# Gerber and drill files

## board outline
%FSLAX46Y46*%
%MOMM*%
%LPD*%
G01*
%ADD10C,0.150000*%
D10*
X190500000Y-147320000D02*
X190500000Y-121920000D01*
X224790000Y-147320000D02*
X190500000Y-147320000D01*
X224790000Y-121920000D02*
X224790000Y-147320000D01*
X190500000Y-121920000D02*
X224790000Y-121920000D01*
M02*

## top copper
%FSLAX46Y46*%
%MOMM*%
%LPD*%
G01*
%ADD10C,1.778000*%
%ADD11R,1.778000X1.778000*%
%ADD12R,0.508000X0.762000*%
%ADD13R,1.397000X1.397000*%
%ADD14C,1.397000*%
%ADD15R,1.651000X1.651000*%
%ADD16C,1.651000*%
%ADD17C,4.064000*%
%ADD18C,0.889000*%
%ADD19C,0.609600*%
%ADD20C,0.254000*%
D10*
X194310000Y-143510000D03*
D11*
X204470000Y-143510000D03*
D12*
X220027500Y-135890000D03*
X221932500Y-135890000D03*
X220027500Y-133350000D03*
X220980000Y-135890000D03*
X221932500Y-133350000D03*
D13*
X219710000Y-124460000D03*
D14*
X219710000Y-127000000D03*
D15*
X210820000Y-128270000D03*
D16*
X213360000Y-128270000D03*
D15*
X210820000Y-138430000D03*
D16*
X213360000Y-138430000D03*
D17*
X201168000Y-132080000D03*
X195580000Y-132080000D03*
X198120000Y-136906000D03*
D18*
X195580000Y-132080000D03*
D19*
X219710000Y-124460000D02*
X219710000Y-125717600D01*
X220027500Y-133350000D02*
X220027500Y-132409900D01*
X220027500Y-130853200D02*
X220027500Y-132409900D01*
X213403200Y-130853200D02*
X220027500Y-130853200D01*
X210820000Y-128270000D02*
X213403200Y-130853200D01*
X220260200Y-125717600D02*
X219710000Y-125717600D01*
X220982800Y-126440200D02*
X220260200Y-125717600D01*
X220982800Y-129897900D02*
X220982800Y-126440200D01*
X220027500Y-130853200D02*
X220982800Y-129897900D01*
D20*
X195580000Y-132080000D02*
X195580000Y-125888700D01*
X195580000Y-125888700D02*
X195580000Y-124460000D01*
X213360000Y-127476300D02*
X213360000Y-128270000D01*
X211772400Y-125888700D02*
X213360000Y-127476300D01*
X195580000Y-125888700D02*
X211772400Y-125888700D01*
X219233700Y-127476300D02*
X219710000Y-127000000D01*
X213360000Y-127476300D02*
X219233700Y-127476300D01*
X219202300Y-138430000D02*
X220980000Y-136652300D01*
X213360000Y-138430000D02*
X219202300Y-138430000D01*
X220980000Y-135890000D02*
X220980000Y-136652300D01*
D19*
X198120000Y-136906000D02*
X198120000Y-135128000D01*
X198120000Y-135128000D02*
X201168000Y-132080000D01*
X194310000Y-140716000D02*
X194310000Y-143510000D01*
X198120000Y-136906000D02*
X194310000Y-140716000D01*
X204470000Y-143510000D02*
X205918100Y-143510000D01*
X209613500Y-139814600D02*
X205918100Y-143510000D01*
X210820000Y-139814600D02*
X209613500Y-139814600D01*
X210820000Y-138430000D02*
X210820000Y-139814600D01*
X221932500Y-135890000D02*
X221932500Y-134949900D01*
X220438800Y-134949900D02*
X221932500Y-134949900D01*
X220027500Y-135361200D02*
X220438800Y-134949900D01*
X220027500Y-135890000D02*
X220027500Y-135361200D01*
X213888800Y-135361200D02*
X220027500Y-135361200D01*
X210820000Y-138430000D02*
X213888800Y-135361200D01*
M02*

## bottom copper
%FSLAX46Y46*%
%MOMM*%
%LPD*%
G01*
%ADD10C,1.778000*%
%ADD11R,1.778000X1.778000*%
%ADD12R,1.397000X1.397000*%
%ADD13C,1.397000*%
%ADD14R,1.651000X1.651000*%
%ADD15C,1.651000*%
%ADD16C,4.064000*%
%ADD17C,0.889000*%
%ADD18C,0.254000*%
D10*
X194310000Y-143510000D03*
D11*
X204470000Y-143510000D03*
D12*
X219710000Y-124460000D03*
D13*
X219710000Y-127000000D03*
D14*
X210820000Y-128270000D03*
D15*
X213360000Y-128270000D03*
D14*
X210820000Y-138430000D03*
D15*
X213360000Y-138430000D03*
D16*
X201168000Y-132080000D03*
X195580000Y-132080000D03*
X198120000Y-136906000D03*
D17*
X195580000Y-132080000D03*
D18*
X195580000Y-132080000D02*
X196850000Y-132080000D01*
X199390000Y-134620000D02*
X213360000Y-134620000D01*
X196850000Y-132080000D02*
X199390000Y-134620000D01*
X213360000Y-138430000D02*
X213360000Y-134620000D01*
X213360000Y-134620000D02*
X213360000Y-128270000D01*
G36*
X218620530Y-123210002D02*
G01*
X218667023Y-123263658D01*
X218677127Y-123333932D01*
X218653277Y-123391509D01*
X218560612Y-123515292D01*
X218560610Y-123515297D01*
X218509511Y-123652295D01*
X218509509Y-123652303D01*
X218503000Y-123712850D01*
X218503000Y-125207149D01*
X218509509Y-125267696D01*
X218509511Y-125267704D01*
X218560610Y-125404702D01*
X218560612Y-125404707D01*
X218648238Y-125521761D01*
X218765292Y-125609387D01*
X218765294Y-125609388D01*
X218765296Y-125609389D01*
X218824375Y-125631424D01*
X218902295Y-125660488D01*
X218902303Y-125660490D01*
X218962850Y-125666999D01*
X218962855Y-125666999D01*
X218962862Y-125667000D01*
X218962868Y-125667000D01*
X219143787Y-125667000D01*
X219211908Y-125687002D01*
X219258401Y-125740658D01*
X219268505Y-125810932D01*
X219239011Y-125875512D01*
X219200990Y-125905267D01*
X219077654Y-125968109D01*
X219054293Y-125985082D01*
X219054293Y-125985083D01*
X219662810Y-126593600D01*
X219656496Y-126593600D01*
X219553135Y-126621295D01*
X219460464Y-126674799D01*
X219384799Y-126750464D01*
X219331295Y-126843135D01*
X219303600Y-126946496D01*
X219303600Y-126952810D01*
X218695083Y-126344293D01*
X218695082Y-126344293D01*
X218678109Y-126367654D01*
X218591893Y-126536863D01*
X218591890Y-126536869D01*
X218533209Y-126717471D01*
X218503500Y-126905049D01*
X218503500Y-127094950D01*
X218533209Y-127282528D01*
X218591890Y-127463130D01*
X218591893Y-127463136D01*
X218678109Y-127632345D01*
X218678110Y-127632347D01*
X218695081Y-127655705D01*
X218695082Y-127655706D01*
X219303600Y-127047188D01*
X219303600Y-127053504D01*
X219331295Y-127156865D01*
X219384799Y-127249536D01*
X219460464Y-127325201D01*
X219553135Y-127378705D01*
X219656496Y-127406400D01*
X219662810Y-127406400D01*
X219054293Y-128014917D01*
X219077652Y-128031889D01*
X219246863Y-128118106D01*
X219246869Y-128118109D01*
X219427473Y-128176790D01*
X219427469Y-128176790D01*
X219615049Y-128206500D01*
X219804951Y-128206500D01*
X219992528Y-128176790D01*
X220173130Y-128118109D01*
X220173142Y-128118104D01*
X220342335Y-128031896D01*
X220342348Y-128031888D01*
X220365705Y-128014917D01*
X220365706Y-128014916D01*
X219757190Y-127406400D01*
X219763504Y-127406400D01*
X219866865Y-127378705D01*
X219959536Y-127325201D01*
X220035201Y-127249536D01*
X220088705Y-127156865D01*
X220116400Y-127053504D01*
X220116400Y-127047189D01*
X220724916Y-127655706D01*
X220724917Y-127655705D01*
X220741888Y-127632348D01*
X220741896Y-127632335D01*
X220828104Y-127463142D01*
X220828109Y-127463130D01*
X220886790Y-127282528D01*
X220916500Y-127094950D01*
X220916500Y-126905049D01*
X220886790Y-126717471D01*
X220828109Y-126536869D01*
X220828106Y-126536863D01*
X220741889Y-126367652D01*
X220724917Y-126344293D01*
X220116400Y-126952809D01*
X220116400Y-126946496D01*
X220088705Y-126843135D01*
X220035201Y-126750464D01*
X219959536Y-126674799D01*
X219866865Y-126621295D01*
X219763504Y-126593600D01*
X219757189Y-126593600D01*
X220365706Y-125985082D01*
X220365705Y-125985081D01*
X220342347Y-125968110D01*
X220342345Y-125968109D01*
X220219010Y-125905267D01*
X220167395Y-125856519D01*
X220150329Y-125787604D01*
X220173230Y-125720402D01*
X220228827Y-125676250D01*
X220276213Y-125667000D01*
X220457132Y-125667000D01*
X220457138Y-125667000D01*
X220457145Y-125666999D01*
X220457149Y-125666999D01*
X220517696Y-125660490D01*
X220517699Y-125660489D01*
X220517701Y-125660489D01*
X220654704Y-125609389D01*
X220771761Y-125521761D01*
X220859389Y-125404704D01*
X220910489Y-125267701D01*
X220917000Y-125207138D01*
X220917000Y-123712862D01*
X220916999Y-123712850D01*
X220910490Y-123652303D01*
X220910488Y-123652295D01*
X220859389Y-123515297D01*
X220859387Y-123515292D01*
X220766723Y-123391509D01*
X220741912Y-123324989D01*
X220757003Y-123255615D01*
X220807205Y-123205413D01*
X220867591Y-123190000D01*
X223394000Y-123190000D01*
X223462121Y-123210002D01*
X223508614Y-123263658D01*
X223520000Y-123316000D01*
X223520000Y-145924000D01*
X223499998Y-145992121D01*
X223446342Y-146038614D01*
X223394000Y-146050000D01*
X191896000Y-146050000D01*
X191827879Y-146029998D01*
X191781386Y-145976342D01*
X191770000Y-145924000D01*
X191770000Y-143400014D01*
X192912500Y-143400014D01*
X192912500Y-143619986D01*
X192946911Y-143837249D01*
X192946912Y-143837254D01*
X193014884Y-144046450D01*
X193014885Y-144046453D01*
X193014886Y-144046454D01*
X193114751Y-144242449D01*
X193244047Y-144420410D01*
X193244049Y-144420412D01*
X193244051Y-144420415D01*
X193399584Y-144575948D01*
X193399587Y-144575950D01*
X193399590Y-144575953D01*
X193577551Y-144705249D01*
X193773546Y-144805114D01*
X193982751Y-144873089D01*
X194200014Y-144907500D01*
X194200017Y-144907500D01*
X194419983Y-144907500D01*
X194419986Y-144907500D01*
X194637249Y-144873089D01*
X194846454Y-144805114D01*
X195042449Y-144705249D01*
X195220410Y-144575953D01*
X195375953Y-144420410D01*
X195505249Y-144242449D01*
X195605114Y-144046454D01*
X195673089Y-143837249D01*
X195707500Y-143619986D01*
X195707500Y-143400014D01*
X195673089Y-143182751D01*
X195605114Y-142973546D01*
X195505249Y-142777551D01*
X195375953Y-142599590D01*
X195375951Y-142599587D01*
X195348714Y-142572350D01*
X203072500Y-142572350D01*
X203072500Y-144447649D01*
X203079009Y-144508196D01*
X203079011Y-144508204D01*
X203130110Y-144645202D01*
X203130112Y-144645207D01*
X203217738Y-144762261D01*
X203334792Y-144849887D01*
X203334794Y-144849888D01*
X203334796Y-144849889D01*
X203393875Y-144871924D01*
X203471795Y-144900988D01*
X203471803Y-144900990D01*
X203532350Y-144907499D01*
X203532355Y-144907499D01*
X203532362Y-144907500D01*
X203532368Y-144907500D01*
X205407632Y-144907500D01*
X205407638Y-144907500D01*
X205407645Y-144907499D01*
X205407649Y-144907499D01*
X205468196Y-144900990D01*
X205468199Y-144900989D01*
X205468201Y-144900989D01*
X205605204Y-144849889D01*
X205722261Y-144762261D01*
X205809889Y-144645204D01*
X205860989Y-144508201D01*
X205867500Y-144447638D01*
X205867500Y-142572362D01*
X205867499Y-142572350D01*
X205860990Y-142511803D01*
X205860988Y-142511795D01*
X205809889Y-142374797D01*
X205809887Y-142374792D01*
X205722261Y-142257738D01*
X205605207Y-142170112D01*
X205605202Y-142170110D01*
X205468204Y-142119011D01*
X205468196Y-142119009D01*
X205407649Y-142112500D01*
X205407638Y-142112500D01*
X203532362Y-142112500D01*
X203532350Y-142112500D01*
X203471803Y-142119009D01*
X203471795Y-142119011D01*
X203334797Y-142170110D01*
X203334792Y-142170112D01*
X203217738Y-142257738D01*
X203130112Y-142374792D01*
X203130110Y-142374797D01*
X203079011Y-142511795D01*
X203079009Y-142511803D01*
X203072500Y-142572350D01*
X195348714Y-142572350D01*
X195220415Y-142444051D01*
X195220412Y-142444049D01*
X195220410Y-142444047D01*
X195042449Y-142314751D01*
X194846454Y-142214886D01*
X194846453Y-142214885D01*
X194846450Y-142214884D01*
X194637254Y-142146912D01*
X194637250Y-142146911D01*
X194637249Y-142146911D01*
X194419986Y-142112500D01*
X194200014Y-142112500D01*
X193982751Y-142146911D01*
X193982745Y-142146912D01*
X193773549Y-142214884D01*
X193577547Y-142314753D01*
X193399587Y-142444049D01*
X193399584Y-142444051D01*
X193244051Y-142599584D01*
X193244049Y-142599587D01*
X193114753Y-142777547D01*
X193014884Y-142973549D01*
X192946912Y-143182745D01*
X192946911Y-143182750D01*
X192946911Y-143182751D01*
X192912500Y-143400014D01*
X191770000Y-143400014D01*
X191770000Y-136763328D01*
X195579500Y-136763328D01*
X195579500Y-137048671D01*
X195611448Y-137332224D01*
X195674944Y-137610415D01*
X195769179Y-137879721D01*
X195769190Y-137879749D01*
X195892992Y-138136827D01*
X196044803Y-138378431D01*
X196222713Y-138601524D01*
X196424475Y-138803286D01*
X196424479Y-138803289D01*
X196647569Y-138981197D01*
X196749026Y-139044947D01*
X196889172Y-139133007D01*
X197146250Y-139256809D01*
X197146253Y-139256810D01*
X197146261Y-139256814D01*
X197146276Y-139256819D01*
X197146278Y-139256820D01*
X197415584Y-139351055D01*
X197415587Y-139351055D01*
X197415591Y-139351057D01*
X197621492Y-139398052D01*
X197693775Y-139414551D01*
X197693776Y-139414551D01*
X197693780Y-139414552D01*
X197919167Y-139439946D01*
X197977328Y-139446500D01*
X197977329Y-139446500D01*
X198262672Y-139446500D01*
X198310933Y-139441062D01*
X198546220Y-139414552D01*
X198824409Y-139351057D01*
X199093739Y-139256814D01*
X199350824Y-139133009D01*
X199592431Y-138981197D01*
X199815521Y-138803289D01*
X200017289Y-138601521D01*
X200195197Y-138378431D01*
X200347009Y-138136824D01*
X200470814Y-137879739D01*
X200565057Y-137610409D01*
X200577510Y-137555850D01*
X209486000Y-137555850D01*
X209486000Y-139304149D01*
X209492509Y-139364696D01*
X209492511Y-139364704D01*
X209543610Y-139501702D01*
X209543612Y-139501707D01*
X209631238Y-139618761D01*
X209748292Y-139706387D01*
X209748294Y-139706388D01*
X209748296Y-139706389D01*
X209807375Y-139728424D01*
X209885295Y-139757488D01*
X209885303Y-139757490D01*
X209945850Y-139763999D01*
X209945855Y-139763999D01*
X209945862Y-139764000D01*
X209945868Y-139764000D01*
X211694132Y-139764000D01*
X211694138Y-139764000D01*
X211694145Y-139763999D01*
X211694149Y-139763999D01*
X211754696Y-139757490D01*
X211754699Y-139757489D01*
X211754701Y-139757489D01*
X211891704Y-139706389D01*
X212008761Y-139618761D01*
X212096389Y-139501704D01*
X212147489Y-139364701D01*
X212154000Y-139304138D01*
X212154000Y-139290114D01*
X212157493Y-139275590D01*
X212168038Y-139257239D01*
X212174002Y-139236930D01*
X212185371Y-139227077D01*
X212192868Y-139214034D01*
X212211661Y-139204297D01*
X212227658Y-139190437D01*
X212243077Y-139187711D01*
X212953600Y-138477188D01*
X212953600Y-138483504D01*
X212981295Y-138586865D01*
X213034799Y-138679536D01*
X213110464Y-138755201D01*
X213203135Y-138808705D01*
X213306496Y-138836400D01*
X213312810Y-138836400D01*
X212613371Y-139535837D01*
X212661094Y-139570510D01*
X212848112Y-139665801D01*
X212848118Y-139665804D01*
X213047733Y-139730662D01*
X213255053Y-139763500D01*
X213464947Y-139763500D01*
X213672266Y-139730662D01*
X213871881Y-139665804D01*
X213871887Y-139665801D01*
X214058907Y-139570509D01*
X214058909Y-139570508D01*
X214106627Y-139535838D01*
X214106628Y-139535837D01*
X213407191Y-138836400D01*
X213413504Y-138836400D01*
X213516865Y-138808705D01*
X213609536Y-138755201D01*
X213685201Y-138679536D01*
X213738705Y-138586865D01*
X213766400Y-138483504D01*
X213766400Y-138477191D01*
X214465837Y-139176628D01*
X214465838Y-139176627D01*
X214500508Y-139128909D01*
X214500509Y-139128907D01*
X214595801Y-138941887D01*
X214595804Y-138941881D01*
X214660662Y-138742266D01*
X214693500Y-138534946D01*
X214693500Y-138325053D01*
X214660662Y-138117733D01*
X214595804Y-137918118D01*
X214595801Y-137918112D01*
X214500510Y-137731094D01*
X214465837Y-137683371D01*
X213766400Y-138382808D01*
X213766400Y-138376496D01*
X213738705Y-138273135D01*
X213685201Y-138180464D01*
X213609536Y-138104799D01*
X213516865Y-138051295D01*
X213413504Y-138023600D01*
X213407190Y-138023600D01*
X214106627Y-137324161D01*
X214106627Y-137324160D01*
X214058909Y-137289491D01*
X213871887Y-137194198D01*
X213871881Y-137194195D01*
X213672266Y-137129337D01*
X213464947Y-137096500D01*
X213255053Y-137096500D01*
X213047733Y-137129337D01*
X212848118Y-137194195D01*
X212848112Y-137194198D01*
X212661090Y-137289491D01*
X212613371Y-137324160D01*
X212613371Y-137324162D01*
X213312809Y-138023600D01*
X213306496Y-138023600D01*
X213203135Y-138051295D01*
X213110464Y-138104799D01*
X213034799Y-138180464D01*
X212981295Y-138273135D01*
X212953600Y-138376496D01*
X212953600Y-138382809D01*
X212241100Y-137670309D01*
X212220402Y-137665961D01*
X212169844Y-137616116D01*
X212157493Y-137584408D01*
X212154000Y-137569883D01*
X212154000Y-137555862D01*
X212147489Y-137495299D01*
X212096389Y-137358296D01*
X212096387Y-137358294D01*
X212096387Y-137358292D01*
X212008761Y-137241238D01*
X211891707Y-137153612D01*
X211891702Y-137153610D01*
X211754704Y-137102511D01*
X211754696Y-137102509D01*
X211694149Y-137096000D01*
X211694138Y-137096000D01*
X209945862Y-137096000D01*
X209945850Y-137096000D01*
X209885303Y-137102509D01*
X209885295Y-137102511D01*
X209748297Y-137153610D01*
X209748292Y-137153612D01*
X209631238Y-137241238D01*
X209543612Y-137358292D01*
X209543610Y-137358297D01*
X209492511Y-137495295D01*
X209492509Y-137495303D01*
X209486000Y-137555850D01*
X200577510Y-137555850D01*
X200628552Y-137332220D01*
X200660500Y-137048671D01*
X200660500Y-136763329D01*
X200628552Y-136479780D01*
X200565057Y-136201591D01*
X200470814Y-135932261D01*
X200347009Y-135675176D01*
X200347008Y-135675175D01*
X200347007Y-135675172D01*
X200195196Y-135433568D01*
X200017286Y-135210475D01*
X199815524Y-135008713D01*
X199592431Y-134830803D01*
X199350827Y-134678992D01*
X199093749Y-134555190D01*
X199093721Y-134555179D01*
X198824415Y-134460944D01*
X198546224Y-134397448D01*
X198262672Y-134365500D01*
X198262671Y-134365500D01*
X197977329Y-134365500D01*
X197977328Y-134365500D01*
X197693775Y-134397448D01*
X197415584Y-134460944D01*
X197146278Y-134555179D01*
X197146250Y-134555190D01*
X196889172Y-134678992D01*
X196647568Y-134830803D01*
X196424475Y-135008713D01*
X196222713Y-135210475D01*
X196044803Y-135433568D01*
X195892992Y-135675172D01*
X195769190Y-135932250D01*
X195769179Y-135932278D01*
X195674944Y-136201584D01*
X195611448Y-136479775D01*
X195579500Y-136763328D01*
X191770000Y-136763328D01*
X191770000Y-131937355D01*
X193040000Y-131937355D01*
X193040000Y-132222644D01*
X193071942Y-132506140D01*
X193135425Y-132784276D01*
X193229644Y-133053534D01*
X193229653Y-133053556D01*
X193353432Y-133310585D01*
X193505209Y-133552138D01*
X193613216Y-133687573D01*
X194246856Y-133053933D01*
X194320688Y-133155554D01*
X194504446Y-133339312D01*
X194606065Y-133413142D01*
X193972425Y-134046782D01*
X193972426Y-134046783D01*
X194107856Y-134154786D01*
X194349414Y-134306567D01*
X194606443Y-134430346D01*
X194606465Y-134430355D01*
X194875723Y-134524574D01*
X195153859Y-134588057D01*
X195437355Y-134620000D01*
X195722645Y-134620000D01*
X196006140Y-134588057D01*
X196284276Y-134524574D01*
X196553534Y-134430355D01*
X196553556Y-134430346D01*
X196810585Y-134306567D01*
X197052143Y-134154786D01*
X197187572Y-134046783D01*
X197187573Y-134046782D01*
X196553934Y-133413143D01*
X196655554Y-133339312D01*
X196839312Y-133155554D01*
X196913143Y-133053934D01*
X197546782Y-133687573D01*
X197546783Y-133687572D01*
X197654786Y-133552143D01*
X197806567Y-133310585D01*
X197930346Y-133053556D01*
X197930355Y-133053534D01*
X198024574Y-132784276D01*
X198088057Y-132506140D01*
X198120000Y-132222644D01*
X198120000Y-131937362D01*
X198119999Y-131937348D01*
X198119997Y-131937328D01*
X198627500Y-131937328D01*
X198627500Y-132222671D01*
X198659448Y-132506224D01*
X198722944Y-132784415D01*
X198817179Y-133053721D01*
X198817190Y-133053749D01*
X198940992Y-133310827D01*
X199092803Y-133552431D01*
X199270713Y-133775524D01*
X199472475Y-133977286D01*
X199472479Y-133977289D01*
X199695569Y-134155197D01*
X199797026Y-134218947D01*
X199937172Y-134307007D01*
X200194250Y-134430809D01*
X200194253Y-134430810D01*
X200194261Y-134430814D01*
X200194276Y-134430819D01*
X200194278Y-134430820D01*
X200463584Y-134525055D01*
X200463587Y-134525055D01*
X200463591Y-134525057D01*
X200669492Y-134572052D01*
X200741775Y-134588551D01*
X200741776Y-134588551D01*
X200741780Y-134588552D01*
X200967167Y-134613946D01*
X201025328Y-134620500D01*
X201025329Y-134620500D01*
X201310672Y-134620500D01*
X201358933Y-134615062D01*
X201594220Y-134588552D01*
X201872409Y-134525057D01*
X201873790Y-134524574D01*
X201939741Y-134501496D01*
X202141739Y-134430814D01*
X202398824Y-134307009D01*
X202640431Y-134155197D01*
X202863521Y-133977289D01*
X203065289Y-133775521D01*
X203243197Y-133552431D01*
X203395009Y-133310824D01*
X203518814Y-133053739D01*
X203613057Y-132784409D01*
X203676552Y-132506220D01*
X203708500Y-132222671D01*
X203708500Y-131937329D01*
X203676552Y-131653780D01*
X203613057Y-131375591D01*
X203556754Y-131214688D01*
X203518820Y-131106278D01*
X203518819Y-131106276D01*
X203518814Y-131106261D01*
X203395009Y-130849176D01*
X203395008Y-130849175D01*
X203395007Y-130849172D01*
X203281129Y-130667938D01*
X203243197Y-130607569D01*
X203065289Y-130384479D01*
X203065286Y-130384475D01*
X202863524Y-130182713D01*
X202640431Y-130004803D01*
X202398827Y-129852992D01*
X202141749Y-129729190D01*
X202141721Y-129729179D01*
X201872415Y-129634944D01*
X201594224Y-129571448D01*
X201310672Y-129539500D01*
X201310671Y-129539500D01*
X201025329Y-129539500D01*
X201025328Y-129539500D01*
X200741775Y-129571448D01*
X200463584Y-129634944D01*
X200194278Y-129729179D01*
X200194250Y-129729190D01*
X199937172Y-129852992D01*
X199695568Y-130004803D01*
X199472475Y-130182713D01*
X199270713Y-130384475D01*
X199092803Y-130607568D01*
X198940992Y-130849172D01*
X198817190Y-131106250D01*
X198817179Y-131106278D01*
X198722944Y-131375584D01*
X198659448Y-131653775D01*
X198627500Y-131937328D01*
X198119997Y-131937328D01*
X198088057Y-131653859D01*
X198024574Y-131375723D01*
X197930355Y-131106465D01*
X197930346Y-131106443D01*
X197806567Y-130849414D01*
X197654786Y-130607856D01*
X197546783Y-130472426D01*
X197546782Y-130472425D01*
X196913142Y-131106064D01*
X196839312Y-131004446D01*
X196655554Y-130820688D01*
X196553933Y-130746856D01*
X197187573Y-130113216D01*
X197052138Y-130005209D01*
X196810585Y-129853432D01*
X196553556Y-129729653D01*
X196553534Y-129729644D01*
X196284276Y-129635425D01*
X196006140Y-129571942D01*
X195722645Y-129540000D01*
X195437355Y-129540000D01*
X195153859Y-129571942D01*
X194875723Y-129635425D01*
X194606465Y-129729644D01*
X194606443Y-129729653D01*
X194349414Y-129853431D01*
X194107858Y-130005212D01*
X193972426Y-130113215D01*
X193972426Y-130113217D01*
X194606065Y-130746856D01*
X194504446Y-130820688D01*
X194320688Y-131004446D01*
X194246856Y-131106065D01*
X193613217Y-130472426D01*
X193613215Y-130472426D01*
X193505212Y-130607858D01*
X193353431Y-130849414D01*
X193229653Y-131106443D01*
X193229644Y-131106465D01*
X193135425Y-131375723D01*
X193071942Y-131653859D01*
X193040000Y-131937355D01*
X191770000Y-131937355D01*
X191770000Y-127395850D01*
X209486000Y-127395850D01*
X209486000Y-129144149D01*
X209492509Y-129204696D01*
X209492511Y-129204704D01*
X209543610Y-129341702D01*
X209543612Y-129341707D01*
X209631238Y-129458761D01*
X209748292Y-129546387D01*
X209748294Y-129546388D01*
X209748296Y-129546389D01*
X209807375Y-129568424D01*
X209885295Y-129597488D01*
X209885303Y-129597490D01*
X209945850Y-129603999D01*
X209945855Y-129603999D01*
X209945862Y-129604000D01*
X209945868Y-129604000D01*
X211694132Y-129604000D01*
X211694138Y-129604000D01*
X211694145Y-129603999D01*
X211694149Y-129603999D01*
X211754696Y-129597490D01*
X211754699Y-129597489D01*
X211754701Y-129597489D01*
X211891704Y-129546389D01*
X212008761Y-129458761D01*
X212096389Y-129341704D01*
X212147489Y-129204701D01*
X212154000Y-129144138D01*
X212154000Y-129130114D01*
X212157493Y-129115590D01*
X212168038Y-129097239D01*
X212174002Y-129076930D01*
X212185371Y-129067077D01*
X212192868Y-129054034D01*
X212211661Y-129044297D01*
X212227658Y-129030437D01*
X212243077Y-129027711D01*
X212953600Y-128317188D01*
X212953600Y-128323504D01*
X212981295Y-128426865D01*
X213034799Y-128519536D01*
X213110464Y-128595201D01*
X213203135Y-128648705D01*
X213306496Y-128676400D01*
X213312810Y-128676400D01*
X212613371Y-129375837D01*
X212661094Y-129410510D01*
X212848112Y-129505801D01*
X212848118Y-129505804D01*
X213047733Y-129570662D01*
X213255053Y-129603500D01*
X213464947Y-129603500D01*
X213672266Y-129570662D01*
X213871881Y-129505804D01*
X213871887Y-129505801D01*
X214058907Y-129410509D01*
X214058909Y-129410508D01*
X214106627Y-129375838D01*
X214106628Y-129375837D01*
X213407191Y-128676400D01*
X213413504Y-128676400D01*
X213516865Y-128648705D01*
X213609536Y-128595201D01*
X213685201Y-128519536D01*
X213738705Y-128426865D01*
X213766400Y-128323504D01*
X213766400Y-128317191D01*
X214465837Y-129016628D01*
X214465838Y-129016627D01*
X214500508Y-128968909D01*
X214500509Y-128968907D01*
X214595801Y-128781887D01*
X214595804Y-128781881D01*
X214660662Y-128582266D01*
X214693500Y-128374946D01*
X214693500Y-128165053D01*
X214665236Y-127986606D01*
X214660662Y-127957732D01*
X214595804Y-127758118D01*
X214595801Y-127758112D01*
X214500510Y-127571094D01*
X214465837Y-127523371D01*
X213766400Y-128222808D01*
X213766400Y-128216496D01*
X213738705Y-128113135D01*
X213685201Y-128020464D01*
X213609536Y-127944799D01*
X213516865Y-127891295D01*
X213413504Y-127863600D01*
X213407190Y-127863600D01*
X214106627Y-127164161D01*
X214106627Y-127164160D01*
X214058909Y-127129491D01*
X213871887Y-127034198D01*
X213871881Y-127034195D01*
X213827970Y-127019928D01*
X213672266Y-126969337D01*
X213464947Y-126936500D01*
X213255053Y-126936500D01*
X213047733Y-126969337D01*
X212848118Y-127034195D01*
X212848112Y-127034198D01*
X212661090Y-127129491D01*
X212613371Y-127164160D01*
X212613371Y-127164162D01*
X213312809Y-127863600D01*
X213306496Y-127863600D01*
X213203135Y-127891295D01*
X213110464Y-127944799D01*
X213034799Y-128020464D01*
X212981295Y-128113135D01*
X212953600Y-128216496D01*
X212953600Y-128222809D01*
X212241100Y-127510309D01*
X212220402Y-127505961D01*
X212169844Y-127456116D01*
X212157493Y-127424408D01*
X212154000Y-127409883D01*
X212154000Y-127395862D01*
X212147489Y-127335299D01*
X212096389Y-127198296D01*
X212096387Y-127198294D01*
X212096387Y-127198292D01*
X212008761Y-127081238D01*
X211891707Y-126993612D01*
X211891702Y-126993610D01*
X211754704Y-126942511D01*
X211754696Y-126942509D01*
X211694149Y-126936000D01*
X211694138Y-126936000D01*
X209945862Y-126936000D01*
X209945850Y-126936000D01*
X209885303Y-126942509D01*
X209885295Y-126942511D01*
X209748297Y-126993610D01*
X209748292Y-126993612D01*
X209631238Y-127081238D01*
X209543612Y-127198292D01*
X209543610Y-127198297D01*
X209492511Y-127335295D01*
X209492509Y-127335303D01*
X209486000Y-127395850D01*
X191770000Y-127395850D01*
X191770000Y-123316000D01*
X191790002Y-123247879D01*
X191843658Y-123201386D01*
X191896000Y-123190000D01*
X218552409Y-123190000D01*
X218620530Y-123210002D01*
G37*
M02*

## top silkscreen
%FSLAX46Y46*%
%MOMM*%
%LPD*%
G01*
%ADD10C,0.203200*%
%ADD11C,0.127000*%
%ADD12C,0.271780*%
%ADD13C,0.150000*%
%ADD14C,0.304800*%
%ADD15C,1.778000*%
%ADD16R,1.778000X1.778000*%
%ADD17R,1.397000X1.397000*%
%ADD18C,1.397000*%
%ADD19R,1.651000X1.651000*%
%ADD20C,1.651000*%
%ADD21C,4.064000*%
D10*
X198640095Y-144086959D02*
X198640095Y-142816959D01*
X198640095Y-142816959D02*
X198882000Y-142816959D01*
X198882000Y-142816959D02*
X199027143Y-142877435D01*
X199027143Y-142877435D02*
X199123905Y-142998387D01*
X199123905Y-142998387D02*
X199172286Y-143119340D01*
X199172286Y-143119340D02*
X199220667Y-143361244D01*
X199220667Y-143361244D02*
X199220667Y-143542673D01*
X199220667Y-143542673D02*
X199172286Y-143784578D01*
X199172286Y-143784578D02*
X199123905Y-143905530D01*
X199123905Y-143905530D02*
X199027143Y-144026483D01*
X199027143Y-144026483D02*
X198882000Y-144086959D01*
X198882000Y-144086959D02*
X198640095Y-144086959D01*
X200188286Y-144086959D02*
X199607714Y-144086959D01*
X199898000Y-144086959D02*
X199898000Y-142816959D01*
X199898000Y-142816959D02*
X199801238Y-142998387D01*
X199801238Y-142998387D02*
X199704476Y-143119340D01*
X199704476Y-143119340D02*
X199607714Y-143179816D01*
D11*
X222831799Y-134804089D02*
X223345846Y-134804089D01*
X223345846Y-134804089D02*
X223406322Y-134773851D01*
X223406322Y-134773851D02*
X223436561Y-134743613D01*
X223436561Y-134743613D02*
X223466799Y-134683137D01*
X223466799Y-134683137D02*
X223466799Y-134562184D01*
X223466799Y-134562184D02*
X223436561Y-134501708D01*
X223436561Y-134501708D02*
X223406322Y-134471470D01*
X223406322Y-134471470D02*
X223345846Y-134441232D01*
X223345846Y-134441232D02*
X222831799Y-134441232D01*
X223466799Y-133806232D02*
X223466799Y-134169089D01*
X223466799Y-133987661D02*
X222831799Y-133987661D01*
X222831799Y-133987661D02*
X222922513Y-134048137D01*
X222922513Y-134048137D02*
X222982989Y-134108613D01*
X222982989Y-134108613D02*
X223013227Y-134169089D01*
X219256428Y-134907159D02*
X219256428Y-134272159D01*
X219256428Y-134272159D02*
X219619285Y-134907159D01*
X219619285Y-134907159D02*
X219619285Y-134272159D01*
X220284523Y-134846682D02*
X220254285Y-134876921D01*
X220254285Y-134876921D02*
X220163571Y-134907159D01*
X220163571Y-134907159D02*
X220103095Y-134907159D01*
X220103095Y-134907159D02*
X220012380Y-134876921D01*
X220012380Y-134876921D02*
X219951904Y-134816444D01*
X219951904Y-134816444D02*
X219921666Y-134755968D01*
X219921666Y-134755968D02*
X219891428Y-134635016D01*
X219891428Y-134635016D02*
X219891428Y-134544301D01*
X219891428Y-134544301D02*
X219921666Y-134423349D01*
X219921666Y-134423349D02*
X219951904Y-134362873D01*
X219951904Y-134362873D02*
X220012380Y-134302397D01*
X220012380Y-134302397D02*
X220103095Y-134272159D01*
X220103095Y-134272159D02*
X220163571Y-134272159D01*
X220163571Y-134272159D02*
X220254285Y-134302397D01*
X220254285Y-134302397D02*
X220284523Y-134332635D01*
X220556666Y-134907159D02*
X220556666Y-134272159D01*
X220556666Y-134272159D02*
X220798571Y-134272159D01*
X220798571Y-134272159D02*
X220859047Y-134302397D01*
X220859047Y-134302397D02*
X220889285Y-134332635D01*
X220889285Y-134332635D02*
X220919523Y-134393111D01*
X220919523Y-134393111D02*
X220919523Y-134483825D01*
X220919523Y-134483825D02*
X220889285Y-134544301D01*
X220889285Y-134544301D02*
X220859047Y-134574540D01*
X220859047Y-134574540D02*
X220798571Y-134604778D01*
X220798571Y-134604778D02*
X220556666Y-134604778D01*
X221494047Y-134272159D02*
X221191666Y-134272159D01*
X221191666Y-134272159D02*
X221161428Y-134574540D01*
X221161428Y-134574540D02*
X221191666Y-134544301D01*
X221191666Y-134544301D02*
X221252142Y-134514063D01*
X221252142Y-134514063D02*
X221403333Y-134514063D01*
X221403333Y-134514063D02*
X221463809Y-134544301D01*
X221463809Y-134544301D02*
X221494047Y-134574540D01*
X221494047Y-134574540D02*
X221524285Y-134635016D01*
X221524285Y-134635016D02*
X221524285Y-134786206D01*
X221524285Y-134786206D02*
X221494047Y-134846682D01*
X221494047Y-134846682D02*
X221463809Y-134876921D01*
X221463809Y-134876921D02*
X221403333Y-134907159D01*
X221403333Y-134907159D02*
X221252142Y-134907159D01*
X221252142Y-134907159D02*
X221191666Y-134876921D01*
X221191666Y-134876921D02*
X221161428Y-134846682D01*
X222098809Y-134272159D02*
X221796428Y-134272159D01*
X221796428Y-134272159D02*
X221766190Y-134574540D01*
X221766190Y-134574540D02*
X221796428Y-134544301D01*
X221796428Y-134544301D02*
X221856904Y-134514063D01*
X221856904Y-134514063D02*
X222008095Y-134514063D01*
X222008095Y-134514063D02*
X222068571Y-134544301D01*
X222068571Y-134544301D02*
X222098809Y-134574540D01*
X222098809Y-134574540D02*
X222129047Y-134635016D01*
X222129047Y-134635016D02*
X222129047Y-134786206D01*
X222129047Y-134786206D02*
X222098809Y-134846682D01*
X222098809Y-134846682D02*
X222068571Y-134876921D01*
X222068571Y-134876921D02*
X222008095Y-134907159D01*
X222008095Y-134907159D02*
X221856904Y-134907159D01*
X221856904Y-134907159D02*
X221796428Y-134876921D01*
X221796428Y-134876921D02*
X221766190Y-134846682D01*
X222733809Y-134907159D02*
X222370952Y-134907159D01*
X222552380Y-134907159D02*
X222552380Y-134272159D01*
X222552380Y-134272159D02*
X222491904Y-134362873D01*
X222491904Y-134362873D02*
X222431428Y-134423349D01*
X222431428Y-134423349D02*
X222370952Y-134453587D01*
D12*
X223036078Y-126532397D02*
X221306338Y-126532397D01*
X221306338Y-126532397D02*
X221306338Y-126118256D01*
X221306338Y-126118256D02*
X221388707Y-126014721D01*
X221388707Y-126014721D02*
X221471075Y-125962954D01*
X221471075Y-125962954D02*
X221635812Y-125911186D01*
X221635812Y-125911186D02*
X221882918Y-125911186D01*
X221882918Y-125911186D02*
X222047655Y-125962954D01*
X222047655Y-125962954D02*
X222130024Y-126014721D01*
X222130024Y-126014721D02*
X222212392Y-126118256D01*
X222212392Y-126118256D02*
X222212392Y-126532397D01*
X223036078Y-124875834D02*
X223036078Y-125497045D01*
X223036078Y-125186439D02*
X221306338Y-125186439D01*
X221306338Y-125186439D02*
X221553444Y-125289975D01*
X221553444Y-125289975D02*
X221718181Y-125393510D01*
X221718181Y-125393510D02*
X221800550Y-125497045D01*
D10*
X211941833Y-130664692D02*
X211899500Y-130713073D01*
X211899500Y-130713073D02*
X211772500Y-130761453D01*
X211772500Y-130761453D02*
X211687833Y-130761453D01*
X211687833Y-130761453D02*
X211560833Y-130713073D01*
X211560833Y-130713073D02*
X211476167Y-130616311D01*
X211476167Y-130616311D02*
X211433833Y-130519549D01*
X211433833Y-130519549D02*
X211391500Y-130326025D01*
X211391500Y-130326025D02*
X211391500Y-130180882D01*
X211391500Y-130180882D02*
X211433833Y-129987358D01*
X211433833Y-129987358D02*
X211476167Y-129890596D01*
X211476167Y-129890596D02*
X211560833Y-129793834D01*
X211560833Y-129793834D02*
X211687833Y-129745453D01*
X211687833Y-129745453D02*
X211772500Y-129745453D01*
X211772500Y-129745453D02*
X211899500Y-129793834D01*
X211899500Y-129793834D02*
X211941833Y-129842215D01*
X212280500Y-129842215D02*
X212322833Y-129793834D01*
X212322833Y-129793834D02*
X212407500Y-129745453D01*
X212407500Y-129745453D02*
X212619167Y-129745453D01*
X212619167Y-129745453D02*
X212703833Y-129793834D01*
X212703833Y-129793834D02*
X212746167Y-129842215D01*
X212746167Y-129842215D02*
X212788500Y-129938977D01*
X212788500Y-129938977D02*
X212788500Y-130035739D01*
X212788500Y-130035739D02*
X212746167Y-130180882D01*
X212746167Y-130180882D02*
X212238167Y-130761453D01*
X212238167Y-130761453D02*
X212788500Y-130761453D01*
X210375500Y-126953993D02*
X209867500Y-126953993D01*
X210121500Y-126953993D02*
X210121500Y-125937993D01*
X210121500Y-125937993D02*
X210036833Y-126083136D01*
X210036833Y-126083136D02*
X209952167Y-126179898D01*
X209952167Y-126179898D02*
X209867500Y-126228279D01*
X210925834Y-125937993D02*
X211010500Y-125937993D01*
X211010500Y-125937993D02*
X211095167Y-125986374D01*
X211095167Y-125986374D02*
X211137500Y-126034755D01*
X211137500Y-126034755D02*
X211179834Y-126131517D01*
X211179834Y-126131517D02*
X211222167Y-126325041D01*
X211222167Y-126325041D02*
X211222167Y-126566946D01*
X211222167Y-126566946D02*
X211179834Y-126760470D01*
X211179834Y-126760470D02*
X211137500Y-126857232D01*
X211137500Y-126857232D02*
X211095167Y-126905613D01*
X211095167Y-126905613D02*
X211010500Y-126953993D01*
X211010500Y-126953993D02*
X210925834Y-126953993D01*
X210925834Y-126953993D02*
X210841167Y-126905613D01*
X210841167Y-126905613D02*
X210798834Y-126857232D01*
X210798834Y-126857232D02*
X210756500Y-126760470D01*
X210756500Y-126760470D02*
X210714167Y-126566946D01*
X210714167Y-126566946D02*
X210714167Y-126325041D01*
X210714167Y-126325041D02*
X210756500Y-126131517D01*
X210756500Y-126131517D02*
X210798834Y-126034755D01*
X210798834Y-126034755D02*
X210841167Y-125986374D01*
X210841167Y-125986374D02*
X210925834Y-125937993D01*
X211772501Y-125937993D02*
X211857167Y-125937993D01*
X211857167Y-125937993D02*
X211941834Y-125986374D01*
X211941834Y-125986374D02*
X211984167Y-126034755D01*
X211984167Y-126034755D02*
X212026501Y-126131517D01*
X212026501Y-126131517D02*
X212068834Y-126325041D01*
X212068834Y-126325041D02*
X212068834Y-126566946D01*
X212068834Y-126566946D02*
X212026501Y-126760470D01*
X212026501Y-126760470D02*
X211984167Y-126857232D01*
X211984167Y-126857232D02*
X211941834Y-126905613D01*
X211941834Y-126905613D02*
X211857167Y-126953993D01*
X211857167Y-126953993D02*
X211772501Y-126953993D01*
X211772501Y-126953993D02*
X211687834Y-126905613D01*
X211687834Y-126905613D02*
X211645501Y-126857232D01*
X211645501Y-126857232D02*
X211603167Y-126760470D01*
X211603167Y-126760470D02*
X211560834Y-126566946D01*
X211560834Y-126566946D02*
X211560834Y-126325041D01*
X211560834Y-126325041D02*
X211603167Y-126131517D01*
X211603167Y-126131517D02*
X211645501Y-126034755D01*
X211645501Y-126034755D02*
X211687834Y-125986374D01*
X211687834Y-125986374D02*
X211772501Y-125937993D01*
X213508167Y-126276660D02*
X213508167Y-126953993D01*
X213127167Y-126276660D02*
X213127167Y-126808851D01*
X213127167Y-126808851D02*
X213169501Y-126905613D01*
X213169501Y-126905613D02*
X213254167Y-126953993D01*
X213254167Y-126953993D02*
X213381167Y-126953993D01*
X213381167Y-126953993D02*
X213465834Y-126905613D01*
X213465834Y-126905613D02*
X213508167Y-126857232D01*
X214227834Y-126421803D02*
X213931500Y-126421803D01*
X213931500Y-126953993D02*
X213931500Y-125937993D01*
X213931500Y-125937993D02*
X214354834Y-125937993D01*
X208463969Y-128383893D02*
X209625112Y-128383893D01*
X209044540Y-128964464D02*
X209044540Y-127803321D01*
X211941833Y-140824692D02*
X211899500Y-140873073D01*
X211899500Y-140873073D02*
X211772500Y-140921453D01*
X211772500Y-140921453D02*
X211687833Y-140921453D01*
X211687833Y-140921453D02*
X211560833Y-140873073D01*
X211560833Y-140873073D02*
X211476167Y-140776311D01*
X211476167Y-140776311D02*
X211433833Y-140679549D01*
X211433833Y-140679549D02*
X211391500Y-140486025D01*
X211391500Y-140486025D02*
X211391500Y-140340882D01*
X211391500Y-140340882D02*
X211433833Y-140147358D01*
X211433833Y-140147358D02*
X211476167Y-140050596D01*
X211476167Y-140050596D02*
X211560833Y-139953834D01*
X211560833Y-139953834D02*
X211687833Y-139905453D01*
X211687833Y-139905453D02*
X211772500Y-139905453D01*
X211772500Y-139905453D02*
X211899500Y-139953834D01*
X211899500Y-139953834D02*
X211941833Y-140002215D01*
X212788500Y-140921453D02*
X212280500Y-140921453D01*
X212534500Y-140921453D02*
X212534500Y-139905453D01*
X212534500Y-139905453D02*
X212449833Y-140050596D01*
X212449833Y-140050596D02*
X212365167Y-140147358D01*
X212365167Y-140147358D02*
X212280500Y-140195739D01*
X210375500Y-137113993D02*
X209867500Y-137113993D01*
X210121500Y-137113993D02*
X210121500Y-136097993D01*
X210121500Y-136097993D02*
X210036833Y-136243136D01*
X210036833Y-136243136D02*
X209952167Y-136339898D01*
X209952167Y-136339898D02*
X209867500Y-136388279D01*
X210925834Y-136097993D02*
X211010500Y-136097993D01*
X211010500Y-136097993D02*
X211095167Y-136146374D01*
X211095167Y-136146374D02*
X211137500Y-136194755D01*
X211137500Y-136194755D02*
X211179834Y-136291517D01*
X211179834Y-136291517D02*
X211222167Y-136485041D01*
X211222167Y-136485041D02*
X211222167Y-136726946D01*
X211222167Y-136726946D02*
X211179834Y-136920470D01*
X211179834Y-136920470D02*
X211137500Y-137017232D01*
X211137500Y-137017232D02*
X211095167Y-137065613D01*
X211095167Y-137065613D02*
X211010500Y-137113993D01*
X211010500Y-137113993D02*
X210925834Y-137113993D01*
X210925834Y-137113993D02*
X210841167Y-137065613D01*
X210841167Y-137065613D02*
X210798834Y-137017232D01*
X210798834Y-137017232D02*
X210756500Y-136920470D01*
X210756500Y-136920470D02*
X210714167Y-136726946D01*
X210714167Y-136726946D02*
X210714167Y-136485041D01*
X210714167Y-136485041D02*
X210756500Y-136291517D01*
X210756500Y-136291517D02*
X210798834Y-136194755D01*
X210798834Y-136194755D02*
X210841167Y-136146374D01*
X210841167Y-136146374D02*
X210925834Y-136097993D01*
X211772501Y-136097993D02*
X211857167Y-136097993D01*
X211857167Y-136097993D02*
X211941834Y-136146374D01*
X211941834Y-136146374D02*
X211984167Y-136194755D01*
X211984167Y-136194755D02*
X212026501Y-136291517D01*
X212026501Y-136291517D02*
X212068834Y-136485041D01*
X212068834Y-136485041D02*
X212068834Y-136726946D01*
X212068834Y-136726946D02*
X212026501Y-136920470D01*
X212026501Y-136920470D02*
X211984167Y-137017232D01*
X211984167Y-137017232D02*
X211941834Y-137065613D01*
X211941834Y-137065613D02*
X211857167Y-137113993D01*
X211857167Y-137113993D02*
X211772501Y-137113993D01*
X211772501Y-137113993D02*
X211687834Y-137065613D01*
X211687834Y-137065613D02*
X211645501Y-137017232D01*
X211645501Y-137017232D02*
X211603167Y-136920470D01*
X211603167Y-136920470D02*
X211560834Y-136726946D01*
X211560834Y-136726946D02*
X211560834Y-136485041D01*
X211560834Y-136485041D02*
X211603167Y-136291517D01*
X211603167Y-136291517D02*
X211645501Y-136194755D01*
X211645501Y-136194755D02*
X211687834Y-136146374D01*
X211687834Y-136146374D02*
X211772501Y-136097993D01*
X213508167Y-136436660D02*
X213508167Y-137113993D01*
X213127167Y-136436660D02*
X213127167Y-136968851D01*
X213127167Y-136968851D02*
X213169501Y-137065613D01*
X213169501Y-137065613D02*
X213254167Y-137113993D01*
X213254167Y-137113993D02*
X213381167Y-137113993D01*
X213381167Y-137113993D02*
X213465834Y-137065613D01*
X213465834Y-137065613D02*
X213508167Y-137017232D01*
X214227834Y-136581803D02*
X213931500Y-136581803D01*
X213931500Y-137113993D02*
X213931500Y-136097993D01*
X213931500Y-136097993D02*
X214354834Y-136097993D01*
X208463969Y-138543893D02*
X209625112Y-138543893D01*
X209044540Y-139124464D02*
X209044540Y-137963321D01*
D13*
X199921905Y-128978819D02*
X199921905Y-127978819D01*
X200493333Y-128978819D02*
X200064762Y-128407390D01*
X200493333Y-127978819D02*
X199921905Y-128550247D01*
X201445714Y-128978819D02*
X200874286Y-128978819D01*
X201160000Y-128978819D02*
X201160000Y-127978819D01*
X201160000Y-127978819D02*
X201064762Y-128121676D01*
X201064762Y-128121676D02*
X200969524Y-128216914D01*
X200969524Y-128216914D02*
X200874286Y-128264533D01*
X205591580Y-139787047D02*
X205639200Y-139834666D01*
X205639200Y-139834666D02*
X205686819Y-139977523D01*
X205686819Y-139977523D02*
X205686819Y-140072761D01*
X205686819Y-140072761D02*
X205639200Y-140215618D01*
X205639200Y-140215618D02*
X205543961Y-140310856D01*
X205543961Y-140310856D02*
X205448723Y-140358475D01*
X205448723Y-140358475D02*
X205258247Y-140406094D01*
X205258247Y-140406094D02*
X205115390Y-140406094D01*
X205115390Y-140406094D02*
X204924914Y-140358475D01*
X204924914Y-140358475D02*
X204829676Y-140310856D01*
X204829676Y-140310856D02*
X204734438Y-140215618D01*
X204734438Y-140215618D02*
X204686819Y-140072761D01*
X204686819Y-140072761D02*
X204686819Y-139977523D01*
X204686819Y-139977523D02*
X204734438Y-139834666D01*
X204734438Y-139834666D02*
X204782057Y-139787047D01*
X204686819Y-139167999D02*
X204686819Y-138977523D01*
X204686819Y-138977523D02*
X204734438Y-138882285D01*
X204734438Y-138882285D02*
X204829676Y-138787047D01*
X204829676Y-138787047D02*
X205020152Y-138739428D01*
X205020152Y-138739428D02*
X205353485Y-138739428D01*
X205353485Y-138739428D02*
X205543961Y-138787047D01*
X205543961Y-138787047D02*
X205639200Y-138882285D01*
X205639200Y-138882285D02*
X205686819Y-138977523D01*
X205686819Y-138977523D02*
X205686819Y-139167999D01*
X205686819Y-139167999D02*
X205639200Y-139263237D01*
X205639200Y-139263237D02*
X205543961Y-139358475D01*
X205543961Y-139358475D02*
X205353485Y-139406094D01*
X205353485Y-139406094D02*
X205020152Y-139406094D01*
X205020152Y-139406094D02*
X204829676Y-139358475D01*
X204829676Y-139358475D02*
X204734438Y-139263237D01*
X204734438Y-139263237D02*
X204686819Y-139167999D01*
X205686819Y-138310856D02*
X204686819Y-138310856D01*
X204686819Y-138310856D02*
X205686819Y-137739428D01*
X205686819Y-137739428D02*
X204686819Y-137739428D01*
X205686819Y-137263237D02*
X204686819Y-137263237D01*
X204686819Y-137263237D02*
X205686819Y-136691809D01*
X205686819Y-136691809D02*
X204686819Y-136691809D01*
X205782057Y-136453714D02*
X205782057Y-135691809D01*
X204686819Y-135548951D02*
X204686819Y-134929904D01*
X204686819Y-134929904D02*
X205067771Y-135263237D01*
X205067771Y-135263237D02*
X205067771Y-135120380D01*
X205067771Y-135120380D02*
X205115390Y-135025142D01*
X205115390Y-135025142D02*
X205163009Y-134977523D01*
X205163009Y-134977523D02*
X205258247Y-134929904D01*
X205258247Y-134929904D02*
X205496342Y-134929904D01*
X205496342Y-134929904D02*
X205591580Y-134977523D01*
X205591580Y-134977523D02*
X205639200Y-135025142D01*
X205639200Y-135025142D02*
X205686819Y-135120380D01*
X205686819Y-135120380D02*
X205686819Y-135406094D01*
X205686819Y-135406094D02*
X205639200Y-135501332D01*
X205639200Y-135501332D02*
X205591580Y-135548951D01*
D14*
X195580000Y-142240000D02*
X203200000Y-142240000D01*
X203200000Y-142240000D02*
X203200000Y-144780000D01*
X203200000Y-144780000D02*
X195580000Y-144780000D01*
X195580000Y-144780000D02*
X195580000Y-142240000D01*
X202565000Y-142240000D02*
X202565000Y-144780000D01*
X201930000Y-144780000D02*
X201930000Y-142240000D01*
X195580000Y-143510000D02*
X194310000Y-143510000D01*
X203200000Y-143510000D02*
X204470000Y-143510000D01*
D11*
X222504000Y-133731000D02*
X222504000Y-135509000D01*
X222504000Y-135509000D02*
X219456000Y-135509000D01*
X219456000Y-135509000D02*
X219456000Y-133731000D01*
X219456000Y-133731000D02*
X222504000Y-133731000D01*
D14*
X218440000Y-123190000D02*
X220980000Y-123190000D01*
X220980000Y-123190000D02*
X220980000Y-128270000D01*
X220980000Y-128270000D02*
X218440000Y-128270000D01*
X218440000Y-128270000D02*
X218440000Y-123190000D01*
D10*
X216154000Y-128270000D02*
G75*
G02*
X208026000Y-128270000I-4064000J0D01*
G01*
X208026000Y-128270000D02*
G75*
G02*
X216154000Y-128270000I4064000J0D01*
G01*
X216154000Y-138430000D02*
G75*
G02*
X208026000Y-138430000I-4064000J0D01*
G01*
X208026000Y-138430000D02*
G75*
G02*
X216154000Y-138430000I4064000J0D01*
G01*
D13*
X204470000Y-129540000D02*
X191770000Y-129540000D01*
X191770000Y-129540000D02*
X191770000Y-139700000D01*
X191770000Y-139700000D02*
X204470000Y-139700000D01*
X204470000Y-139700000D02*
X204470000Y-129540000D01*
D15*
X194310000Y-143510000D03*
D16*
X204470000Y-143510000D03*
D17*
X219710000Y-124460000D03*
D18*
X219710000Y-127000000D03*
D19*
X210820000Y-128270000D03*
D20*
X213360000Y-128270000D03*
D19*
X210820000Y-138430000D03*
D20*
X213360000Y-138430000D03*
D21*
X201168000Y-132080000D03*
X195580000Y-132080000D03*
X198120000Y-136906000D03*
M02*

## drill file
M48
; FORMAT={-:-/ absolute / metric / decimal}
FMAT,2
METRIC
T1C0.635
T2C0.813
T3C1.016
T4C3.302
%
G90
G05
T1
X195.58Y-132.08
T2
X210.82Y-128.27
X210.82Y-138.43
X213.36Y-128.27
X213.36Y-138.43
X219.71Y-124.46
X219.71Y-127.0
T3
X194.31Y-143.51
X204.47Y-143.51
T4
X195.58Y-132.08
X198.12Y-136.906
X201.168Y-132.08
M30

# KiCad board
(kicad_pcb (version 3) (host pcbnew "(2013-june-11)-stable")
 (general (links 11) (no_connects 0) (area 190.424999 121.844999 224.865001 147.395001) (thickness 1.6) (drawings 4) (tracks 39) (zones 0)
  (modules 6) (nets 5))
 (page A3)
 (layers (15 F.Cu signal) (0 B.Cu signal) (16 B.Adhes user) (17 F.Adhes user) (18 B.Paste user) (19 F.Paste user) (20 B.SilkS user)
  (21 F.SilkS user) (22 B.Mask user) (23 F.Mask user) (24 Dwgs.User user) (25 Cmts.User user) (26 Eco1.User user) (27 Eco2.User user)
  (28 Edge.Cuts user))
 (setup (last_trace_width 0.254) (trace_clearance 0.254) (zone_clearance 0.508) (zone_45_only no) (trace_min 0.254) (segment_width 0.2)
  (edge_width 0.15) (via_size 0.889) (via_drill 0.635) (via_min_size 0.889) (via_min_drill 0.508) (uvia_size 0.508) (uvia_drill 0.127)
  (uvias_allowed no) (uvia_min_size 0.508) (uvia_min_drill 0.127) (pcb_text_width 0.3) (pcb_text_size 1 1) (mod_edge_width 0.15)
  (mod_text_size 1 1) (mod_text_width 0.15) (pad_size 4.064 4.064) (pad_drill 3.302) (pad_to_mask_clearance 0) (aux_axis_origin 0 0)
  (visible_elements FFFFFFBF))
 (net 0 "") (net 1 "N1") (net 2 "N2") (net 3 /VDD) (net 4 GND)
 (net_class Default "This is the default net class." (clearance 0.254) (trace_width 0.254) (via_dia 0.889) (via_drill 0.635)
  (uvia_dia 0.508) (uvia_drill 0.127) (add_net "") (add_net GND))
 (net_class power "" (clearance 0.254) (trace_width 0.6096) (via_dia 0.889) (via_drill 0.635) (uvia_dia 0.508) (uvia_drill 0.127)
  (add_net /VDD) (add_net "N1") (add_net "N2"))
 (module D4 (layer F.Cu) (at 199.39 143.51)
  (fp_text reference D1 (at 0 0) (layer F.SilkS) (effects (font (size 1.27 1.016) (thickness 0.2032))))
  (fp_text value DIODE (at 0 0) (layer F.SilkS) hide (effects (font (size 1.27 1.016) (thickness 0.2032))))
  (fp_line (start -3.81 -1.27) (end 3.81 -1.27) (layer F.SilkS) (width 0.3048))
  (fp_line (start 3.81 -1.27) (end 3.81 1.27) (layer F.SilkS) (width 0.3048))
  (fp_line (start 3.81 1.27) (end -3.81 1.27) (layer F.SilkS) (width 0.3048))
  (fp_line (start -3.81 1.27) (end -3.81 -1.27) (layer F.SilkS) (width 0.3048))
  (fp_line (start 3.175 -1.27) (end 3.175 1.27) (layer F.SilkS) (width 0.3048))
  (fp_line (start 2.54 1.27) (end 2.54 -1.27) (layer F.SilkS) (width 0.3048))
  (fp_line (start -3.81 0) (end -5.08 0) (layer F.SilkS) (width 0.3048))
  (fp_line (start 3.81 0) (end 5.08 0) (layer F.SilkS) (width 0.3048))
  (pad 1 thru_hole circle (at -5.08 0) (size 1.778 1.778) (drill 1.016) (layers *.Cu *.Mask F.SilkS) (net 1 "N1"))
  (pad 2 thru_hole rect (at 5.08 0) (size 1.778 1.778) (drill 1.016) (layers *.Cu *.Mask F.SilkS) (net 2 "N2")))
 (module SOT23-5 (layer F.Cu) (at 220.98 134.62)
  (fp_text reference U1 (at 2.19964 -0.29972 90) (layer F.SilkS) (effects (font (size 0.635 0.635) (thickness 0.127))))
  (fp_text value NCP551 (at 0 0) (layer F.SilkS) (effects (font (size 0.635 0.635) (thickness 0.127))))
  (fp_line (start 1.524 -0.889) (end 1.524 0.889) (layer F.SilkS) (width 0.127))
  (fp_line (start 1.524 0.889) (end -1.524 0.889) (layer F.SilkS) (width 0.127))
  (fp_line (start -1.524 0.889) (end -1.524 -0.889) (layer F.SilkS) (width 0.127))
  (fp_line (start -1.524 -0.889) (end 1.524 -0.889) (layer F.SilkS) (width 0.127))
  (pad 1 smd rect (at -0.9525 1.27) (size 0.508 0.762) (layers F.Cu F.Paste F.Mask) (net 2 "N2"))
  (pad 3 smd rect (at 0.9525 1.27) (size 0.508 0.762) (layers F.Cu F.Paste F.Mask) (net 2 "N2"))
  (pad 5 smd rect (at -0.9525 -1.27) (size 0.508 0.762) (layers F.Cu F.Paste F.Mask) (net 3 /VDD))
  (pad 2 smd rect (at 0 1.27) (size 0.508 0.762) (layers F.Cu F.Paste F.Mask) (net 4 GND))
  (pad 4 smd rect (at 0.9525 -1.27) (size 0.508 0.762) (layers F.Cu F.Paste F.Mask)))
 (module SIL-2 (layer F.Cu) (at 219.71 125.73 270)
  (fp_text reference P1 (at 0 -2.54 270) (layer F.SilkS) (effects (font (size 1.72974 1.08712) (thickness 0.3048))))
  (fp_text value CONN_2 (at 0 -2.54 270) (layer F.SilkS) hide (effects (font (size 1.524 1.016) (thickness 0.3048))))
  (fp_line (start -2.54 1.27) (end -2.54 -1.27) (layer F.SilkS) (width 0.3048))
  (fp_line (start -2.54 -1.27) (end 2.54 -1.27) (layer F.SilkS) (width 0.3048))
  (fp_line (start 2.54 -1.27) (end 2.54 1.27) (layer F.SilkS) (width 0.3048))
  (fp_line (start 2.54 1.27) (end -2.54 1.27) (layer F.SilkS) (width 0.3048))
  (pad 1 thru_hole rect (at -1.27 0 270) (size 1.397 1.397) (drill 0.8128) (layers *.Cu *.Mask F.SilkS) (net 3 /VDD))
  (pad 2 thru_hole circle (at 1.27 0 270) (size 1.397 1.397) (drill 0.8128) (layers *.Cu *.Mask F.SilkS) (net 4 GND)))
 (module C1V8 (layer F.Cu) (at 212.09 128.27)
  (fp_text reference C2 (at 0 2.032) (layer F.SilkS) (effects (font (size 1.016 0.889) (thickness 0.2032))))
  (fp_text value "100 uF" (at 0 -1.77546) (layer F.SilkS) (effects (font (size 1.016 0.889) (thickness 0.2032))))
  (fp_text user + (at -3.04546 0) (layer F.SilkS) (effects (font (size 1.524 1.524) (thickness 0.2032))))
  (fp_circle (center 0 0) (end 4.064 0) (layer F.SilkS) (width 0.2032))
  (pad 1 thru_hole rect (at -1.27 0) (size 1.651 1.651) (drill 0.8128) (layers *.Cu *.Mask F.SilkS) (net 3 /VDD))
  (pad 2 thru_hole circle (at 1.27 0) (size 1.651 1.651) (drill 0.8128) (layers *.Cu *.Mask F.SilkS) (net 4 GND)))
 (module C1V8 (layer F.Cu) (at 212.09 138.43)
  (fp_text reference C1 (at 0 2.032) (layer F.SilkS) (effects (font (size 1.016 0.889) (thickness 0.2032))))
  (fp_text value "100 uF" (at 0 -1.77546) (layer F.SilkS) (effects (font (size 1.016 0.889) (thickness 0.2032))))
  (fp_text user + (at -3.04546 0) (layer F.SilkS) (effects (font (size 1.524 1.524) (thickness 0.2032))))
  (fp_circle (center 0 0) (end 4.064 0) (layer F.SilkS) (width 0.2032))
  (pad 1 thru_hole rect (at -1.27 0) (size 1.651 1.651) (drill 0.8128) (layers *.Cu *.Mask F.SilkS) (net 2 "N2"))
  (pad 2 thru_hole circle (at 1.27 0) (size 1.651 1.651) (drill 0.8128) (layers *.Cu *.Mask F.SilkS) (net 4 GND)))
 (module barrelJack (layer F.Cu) (at 198.12 134.62 270)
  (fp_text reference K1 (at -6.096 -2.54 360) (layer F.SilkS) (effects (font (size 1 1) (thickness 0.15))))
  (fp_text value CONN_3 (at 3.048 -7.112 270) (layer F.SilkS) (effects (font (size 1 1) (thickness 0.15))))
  (fp_line (start -5.08 -6.35) (end -5.08 6.35) (layer F.SilkS) (width 0.15))
  (fp_line (start -5.08 6.35) (end 5.08 6.35) (layer F.SilkS) (width 0.15))
  (fp_line (start 5.08 6.35) (end 5.08 -6.35) (layer F.SilkS) (width 0.15))
  (fp_line (start 5.08 -6.35) (end -5.08 -6.35) (layer F.SilkS) (width 0.15))
  (pad 1 thru_hole circle (at -2.54 -3.048 270) (size 4.064 4.064) (drill 3.302) (layers *.Cu *.Mask F.SilkS) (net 1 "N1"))
  (pad 2 thru_hole circle (at -2.54 2.54 270) (size 4.064 4.064) (drill 3.302) (layers *.Cu *.Mask F.SilkS) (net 4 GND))
  (pad 3 thru_hole circle (at 2.286 0 270) (size 4.064 4.064) (drill 3.302) (layers *.Cu *.Mask F.SilkS) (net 1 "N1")))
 (gr_line (start 190.5 147.32) (end 190.5 121.92) (angle 90) (layer Edge.Cuts) (width 0.15))
 (gr_line (start 224.79 147.32) (end 190.5 147.32) (angle 90) (layer Edge.Cuts) (width 0.15))
 (gr_line (start 224.79 121.92) (end 224.79 147.32) (angle 90) (layer Edge.Cuts) (width 0.15))
 (gr_line (start 190.5 121.92) (end 224.79 121.92) (angle 90) (layer Edge.Cuts) (width 0.15))
 (segment (start 219.71 124.46) (end 219.71 125.7176) (width 0.6096) (layer F.Cu) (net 3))
 (segment (start 220.0275 133.35) (end 220.0275 132.4099) (width 0.6096) (layer F.Cu) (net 3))
 (segment (start 220.0275 130.8532) (end 220.0275 132.4099) (width 0.6096) (layer F.Cu) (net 3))
 (segment (start 213.4032 130.8532) (end 220.0275 130.8532) (width 0.6096) (layer F.Cu) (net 3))
 (segment (start 210.82 128.27) (end 213.4032 130.8532) (width 0.6096) (layer F.Cu) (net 3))
 (segment (start 220.2602 125.7176) (end 219.71 125.7176) (width 0.6096) (layer F.Cu) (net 3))
 (segment (start 220.9828 126.4402) (end 220.2602 125.7176) (width 0.6096) (layer F.Cu) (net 3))
 (segment (start 220.9828 129.8979) (end 220.9828 126.4402) (width 0.6096) (layer F.Cu) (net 3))
 (segment (start 220.0275 130.8532) (end 220.9828 129.8979) (width 0.6096) (layer F.Cu) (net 3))
 (segment (start 195.58 132.08) (end 196.85 132.08) (width 0.254) (layer B.Cu) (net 4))
 (segment (start 199.39 134.62) (end 213.36 134.62) (width 0.254) (layer B.Cu) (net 4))
 (segment (start 196.85 132.08) (end 199.39 134.62) (width 0.254) (layer B.Cu) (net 4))
 (via (at 195.58 132.08) (size 0.889) (layers F.Cu B.Cu) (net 4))
 (segment (start 213.36 138.43) (end 213.36 134.62) (width 0.254) (layer B.Cu) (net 4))
 (segment (start 213.36 134.62) (end 213.36 128.27) (width 0.254) (layer B.Cu) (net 4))
 (segment (start 195.58 132.08) (end 195.58 125.8887) (width 0.254) (layer F.Cu) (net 4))
 (segment (start 195.58 125.8887) (end 195.58 124.46) (width 0.254) (layer F.Cu) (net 4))
 (segment (start 213.36 127.4763) (end 213.36 128.27) (width 0.254) (layer F.Cu) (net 4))
 (segment (start 211.7724 125.8887) (end 213.36 127.4763) (width 0.254) (layer F.Cu) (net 4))
 (segment (start 195.58 125.8887) (end 211.7724 125.8887) (width 0.254) (layer F.Cu) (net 4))
 (segment (start 219.2337 127.4763) (end 219.71 127) (width 0.254) (layer F.Cu) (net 4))
 (segment (start 213.36 127.4763) (end 219.2337 127.4763) (width 0.254) (layer F.Cu) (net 4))
 (segment (start 219.2023 138.43) (end 220.98 136.6523) (width 0.254) (layer F.Cu) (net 4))
 (segment (start 213.36 138.43) (end 219.2023 138.43) (width 0.254) (layer F.Cu) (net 4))
 (segment (start 220.98 135.89) (end 220.98 136.6523) (width 0.254) (layer F.Cu) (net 4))
 (segment (start 198.12 136.906) (end 198.12 135.128) (width 0.6096) (layer F.Cu) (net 1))
 (segment (start 198.12 135.128) (end 201.168 132.08) (width 0.6096) (layer F.Cu) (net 1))
 (segment (start 194.31 140.716) (end 194.31 143.51) (width 0.6096) (layer F.Cu) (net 1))
 (segment (start 198.12 136.906) (end 194.31 140.716) (width 0.6096) (layer F.Cu) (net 1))
 (segment (start 204.47 143.51) (end 205.9181 143.51) (width 0.6096) (layer F.Cu) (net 2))
 (segment (start 209.6135 139.8146) (end 205.9181 143.51) (width 0.6096) (layer F.Cu) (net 2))
 (segment (start 210.82 139.8146) (end 209.6135 139.8146) (width 0.6096) (layer F.Cu) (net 2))
 (segment (start 210.82 138.43) (end 210.82 139.8146) (width 0.6096) (layer F.Cu) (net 2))
 (segment (start 221.9325 135.89) (end 221.9325 134.9499) (width 0.6096) (layer F.Cu) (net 2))
 (segment (start 220.4388 134.9499) (end 221.9325 134.9499) (width 0.6096) (layer F.Cu) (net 2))
 (segment (start 220.0275 135.3612) (end 220.4388 134.9499) (width 0.6096) (layer F.Cu) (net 2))
 (segment (start 220.0275 135.89) (end 220.0275 135.3612) (width 0.6096) (layer F.Cu) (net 2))
 (segment (start 213.8888 135.3612) (end 220.0275 135.3612) (width 0.6096) (layer F.Cu) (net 2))
 (segment (start 210.82 138.43) (end 213.8888 135.3612) (width 0.6096) (layer F.Cu) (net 2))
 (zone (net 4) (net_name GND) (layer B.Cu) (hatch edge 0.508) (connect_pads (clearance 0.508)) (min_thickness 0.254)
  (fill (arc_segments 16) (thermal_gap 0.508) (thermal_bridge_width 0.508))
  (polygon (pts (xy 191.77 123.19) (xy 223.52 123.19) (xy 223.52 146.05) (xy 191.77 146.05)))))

